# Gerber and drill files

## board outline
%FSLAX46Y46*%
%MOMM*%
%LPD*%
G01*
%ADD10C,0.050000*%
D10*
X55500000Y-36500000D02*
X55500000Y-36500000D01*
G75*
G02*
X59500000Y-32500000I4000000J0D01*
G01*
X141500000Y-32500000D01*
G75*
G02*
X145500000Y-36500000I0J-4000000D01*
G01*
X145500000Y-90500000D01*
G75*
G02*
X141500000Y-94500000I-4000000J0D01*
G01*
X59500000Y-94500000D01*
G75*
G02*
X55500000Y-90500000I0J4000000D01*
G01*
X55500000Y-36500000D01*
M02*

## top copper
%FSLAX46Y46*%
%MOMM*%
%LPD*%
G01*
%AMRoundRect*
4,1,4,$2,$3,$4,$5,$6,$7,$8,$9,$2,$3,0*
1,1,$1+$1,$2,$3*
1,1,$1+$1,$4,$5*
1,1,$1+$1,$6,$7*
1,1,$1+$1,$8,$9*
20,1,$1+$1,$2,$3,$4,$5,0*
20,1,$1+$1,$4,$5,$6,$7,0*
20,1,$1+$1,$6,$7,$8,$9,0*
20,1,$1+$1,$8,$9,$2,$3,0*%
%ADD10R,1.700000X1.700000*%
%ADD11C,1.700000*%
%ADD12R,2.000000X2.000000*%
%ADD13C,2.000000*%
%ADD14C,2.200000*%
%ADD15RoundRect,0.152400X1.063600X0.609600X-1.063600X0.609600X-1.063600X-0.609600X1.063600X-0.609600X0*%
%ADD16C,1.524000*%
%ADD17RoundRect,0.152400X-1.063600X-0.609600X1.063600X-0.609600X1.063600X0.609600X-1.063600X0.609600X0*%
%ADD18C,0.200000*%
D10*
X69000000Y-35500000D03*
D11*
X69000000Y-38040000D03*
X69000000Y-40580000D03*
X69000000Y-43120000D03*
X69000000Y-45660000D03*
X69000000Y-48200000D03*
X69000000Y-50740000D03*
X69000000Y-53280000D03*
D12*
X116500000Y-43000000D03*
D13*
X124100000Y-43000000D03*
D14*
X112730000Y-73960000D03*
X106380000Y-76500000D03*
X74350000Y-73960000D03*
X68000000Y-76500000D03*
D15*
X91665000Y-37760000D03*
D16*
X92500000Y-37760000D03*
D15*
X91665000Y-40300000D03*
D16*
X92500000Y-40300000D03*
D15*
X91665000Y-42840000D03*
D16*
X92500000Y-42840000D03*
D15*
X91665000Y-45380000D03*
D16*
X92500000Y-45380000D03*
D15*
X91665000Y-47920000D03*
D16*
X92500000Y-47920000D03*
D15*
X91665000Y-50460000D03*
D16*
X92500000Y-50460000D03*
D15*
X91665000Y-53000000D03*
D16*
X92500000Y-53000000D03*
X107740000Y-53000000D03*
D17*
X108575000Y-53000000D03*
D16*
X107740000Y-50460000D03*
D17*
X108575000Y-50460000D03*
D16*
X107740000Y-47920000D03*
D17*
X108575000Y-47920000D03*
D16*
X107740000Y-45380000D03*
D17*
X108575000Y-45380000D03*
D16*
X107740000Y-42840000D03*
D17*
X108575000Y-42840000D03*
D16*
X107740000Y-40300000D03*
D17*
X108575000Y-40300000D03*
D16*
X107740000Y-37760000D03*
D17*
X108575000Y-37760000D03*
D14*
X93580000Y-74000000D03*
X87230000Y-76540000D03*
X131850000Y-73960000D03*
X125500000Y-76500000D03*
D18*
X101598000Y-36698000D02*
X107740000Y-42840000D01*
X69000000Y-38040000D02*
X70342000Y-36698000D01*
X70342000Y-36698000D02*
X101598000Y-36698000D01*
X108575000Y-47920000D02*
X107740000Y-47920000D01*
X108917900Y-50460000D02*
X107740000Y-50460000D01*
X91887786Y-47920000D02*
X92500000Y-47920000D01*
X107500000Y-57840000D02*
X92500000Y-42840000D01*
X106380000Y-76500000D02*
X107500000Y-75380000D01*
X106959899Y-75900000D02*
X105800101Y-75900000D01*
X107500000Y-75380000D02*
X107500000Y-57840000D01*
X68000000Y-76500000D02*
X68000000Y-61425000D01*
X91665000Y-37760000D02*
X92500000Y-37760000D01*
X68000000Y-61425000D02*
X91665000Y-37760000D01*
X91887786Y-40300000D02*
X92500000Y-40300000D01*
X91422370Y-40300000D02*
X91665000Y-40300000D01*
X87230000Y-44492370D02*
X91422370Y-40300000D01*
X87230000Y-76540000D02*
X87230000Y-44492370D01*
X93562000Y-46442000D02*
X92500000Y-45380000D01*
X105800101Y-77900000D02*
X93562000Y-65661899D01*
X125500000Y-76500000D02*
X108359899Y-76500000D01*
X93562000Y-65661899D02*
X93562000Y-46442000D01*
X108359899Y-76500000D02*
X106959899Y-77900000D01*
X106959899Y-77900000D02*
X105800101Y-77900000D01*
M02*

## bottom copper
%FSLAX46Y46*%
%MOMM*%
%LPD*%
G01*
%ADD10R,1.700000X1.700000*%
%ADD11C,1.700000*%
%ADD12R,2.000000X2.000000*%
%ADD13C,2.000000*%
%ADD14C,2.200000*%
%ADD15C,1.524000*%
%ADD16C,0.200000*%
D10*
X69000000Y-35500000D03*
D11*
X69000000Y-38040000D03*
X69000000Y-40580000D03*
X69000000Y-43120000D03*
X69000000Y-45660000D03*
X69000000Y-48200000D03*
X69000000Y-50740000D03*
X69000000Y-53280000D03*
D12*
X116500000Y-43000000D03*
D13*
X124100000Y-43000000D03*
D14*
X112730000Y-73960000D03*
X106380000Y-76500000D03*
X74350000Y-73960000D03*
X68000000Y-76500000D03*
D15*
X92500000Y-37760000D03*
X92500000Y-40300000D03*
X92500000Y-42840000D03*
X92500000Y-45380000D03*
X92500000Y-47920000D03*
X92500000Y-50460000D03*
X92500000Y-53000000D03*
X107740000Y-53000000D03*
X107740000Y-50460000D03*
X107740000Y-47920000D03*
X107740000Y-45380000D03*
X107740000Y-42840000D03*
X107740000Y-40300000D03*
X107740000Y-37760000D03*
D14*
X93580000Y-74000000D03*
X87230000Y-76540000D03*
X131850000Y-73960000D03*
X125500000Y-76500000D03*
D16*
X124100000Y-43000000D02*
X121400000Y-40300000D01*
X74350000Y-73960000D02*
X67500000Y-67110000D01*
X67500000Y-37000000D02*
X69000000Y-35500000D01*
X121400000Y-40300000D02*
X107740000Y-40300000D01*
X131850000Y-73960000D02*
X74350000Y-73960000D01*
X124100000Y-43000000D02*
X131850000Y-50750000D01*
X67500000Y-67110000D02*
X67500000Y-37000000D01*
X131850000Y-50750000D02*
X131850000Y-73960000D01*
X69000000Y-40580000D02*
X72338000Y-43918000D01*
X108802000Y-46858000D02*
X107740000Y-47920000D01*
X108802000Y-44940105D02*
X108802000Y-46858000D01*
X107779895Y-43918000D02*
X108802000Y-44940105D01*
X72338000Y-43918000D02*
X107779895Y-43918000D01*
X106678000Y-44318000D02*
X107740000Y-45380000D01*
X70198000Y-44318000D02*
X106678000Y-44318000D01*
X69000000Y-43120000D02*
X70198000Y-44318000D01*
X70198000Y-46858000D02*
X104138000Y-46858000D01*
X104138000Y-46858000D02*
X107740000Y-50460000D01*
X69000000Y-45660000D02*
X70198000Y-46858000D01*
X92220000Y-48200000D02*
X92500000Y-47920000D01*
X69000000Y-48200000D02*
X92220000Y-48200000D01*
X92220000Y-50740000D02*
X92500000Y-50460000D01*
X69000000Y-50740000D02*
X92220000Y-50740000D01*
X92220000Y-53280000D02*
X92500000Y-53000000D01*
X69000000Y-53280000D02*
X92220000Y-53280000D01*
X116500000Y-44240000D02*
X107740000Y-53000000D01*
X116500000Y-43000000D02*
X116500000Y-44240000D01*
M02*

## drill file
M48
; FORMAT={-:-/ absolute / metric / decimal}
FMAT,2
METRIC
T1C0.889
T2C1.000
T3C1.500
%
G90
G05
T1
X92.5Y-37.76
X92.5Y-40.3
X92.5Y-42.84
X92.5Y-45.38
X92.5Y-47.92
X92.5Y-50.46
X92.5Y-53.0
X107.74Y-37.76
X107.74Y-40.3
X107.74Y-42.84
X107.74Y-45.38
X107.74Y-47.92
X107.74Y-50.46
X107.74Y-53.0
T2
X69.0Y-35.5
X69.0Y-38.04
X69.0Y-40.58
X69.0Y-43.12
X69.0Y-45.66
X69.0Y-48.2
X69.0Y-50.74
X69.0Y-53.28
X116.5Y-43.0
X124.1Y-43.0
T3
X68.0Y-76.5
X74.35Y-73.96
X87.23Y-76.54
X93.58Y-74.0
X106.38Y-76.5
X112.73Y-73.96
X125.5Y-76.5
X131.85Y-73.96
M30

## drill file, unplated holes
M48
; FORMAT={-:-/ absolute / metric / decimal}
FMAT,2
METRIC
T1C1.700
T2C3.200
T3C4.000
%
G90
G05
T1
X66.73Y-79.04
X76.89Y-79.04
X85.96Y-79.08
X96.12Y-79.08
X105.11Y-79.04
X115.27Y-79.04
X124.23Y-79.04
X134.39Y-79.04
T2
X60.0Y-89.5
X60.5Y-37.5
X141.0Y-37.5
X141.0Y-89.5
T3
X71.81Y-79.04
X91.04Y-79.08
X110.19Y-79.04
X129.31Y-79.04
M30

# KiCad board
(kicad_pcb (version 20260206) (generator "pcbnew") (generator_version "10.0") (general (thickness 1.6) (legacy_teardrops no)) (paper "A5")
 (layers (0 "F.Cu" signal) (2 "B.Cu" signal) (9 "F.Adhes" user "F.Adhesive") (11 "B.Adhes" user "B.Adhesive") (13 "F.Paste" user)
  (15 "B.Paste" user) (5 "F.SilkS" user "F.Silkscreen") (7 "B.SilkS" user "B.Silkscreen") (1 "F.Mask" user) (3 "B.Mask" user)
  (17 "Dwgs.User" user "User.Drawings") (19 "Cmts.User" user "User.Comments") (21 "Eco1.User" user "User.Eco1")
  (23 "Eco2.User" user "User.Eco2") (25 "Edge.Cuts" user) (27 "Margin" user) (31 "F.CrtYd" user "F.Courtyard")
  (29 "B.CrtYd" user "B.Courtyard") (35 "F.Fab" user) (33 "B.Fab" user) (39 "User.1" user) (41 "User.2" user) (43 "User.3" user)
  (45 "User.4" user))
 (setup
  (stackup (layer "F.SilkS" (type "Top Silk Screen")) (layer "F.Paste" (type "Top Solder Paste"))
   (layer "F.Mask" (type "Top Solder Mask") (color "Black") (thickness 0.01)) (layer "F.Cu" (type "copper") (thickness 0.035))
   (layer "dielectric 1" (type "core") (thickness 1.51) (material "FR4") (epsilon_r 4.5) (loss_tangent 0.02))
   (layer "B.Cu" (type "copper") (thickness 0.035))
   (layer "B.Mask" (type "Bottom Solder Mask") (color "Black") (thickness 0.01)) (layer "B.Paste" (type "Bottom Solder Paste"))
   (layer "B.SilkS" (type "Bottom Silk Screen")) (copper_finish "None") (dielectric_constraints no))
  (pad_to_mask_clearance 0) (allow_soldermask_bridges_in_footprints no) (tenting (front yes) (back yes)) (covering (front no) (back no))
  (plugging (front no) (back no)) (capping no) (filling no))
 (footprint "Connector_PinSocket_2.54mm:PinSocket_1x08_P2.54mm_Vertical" (layer "F.Cu") (at 69 35.5)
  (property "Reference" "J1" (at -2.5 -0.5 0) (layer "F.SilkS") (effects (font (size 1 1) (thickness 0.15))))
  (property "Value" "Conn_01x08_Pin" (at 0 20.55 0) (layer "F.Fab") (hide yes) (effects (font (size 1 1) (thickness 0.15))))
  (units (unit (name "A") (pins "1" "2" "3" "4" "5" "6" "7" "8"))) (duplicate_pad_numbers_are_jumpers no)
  (pad "1" thru_hole rect (at 0 0) (size 1.7 1.7) (drill 1) (layers "*.Cu" "*.Mask") (remove_unused_layers no) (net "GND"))
  (pad "2" thru_hole circle (at 0 2.54) (size 1.7 1.7) (drill 1) (layers "*.Cu" "*.Mask") (remove_unused_layers no) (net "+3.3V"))
  (pad "3" thru_hole circle (at 0 5.08) (size 1.7 1.7) (drill 1) (layers "*.Cu" "*.Mask") (remove_unused_layers no) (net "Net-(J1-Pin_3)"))
  (pad "4" thru_hole circle (at 0 7.62) (size 1.7 1.7) (drill 1) (layers "*.Cu" "*.Mask") (remove_unused_layers no) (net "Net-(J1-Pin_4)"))
  (pad "5" thru_hole circle (at 0 10.16) (size 1.7 1.7) (drill 1) (layers "*.Cu" "*.Mask") (remove_unused_layers no) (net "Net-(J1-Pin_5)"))
  (pad "6" thru_hole circle (at 0 12.7) (size 1.7 1.7) (drill 1) (layers "*.Cu" "*.Mask") (remove_unused_layers no) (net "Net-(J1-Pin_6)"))
  (pad "7" thru_hole circle (at 0 15.24) (size 1.7 1.7) (drill 1) (layers "*.Cu" "*.Mask") (remove_unused_layers no) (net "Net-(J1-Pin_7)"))
  (pad "8" thru_hole circle (at 0 17.78) (size 1.7 1.7) (drill 1) (layers "*.Cu" "*.Mask") (remove_unused_layers no) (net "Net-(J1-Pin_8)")))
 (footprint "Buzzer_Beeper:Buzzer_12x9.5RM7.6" (layer "F.Cu") (at 116.5 43)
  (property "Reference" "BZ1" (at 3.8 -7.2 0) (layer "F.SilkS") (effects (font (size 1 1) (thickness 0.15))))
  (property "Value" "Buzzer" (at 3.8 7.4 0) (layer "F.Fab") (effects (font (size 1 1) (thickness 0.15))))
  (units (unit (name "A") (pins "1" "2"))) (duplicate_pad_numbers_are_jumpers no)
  (pad "1" thru_hole rect (at 0 0) (size 2 2) (drill 1) (layers "*.Cu" "*.Mask") (remove_unused_layers no) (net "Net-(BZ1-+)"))
  (pad "2" thru_hole circle (at 7.6 0) (size 2 2) (drill 1) (layers "*.Cu" "*.Mask") (remove_unused_layers no) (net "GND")))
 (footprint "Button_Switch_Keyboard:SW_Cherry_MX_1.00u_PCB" (layer "F.Cu") (at 112.73 73.96)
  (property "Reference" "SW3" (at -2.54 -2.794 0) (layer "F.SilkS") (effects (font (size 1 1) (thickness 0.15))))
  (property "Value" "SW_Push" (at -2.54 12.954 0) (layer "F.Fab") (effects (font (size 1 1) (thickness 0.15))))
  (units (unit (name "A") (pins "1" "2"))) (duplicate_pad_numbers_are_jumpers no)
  (pad "" np_thru_hole circle (at -7.62 5.08) (size 1.7 1.7) (drill 1.7) (layers "*.Cu" "*.Mask"))
  (pad "" np_thru_hole circle (at -2.54 5.08) (size 4 4) (drill 4) (layers "*.Cu" "*.Mask"))
  (pad "" np_thru_hole circle (at 2.54 5.08) (size 1.7 1.7) (drill 1.7) (layers "*.Cu" "*.Mask"))
  (pad "1" thru_hole circle (at 0 0) (size 2.2 2.2) (drill 1.5) (layers "*.Cu" "*.Mask") (remove_unused_layers no) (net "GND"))
  (pad "2" thru_hole circle (at -6.35 2.54) (size 2.2 2.2) (drill 1.5) (layers "*.Cu" "*.Mask") (remove_unused_layers no)
   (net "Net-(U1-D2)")))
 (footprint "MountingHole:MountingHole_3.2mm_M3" (layer "F.Cu") (at 141 89.5)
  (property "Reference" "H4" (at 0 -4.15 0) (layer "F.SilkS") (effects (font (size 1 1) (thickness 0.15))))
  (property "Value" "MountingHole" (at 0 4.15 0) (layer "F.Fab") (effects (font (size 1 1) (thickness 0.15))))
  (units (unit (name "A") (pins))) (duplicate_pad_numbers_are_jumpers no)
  (pad "" np_thru_hole circle (at 0 0) (size 3.2 3.2) (drill 3.2) (layers "*.Cu" "*.Mask")))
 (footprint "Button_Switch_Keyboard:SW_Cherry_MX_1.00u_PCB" (layer "F.Cu") (at 74.35 73.96)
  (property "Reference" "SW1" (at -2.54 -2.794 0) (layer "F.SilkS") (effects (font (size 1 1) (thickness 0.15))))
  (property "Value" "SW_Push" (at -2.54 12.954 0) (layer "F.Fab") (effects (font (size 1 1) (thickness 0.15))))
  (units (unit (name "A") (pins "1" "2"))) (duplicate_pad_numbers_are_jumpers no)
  (pad "" np_thru_hole circle (at -7.62 5.08) (size 1.7 1.7) (drill 1.7) (layers "*.Cu" "*.Mask"))
  (pad "" np_thru_hole circle (at -2.54 5.08) (size 4 4) (drill 4) (layers "*.Cu" "*.Mask"))
  (pad "" np_thru_hole circle (at 2.54 5.08) (size 1.7 1.7) (drill 1.7) (layers "*.Cu" "*.Mask"))
  (pad "1" thru_hole circle (at 0 0) (size 2.2 2.2) (drill 1.5) (layers "*.Cu" "*.Mask") (remove_unused_layers no) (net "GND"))
  (pad "2" thru_hole circle (at -6.35 2.54) (size 2.2 2.2) (drill 1.5) (layers "*.Cu" "*.Mask") (remove_unused_layers no)
   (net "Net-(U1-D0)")))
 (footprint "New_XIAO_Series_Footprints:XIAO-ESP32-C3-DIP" (layer "F.Cu") (at 100.12 45.38 90)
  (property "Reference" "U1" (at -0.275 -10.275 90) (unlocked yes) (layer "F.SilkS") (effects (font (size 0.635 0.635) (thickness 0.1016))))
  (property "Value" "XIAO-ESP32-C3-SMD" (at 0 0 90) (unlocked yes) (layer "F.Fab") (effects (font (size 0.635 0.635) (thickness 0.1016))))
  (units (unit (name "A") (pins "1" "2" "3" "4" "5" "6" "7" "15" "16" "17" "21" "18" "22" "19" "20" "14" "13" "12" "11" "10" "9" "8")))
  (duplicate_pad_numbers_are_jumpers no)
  (pad "1" smd roundrect (at 7.62 -8.455 180) (size 2.432 1.524) (layers "F.Cu" "F.Mask") (roundrect_rratio 0.1) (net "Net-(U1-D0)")
   (thermal_bridge_angle 45))
  (pad "1" thru_hole circle (at 7.62 -7.62 180) (size 1.524 1.524) (drill 0.889) (layers "*.Cu" "*.Mask") (remove_unused_layers no)
   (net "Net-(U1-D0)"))
  (pad "2" smd roundrect (at 5.08 -8.455 180) (size 2.432 1.524) (layers "F.Cu" "F.Mask") (roundrect_rratio 0.1) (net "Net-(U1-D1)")
   (thermal_bridge_angle 45))
  (pad "2" thru_hole circle (at 5.08 -7.62 180) (size 1.524 1.524) (drill 0.889) (layers "*.Cu" "*.Mask") (remove_unused_layers no)
   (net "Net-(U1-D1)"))
  (pad "3" smd roundrect (at 2.54 -8.455 180) (size 2.432 1.524) (layers "F.Cu" "F.Mask") (roundrect_rratio 0.1) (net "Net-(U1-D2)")
   (thermal_bridge_angle 45))
  (pad "3" thru_hole circle (at 2.54 -7.62 180) (size 1.524 1.524) (drill 0.889) (layers "*.Cu" "*.Mask") (remove_unused_layers no)
   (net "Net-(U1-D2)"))
  (pad "4" smd roundrect (at 0 -8.455 180) (size 2.432 1.524) (layers "F.Cu" "F.Mask") (roundrect_rratio 0.1) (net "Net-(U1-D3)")
   (thermal_bridge_angle 45))
  (pad "4" thru_hole circle (at 0 -7.62 180) (size 1.524 1.524) (drill 0.889) (layers "*.Cu" "*.Mask") (remove_unused_layers no)
   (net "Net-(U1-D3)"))
  (pad "5" smd roundrect (at -2.54 -8.455 180) (size 2.432 1.524) (layers "F.Cu" "F.Mask") (roundrect_rratio 0.1) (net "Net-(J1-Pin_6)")
   (thermal_bridge_angle 45))
  (pad "5" thru_hole circle (at -2.54 -7.62 180) (size 1.524 1.524) (drill 0.889) (layers "*.Cu" "*.Mask") (remove_unused_layers no)
   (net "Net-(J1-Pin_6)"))
  (pad "6" smd roundrect (at -5.08 -8.455 180) (size 2.432 1.524) (layers "F.Cu" "F.Mask") (roundrect_rratio 0.1) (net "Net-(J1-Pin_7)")
   (thermal_bridge_angle 45))
  (pad "6" thru_hole circle (at -5.08 -7.62 180) (size 1.524 1.524) (drill 0.889) (layers "*.Cu" "*.Mask") (remove_unused_layers no)
   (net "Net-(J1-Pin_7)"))
  (pad "7" smd roundrect (at -7.62 -8.455 180) (size 2.432 1.524) (layers "F.Cu" "F.Mask") (roundrect_rratio 0.1) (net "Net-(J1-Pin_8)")
   (thermal_bridge_angle 45))
  (pad "7" thru_hole circle (at -7.62 -7.62 180) (size 1.524 1.524) (drill 0.889) (layers "*.Cu" "*.Mask") (remove_unused_layers no)
   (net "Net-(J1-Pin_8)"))
  (pad "8" thru_hole circle (at -7.62 7.62) (size 1.524 1.524) (drill 0.889) (layers "*.Cu" "*.Mask") (remove_unused_layers no)
   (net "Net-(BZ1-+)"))
  (pad "8" smd roundrect (at -7.62 8.455) (size 2.432 1.524) (layers "F.Cu" "F.Mask") (roundrect_rratio 0.1) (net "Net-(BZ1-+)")
   (thermal_bridge_angle 45))
  (pad "9" thru_hole circle (at -5.08 7.62) (size 1.524 1.524) (drill 0.889) (layers "*.Cu" "*.Mask") (remove_unused_layers no)
   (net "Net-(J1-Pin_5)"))
  (pad "9" smd roundrect (at -5.08 8.455) (size 2.432 1.524) (layers "F.Cu" "F.Mask") (roundrect_rratio 0.1) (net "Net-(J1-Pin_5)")
   (thermal_bridge_angle 45))
  (pad "10" thru_hole circle (at -2.54 7.62) (size 1.524 1.524) (drill 0.889) (layers "*.Cu" "*.Mask") (remove_unused_layers no)
   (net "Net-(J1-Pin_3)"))
  (pad "10" smd roundrect (at -2.54 8.455) (size 2.432 1.524) (layers "F.Cu" "F.Mask") (roundrect_rratio 0.1) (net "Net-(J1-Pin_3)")
   (thermal_bridge_angle 45))
  (pad "11" thru_hole circle (at 0 7.62) (size 1.524 1.524) (drill 0.889) (layers "*.Cu" "*.Mask") (remove_unused_layers no)
   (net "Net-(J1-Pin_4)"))
  (pad "11" smd roundrect (at 0 8.455) (size 2.432 1.524) (layers "F.Cu" "F.Mask") (roundrect_rratio 0.1) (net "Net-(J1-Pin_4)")
   (thermal_bridge_angle 45))
  (pad "12" thru_hole circle (at 2.54 7.62) (size 1.524 1.524) (drill 0.889) (layers "*.Cu" "*.Mask") (remove_unused_layers no)
   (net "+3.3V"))
  (pad "12" smd roundrect (at 2.54 8.455) (size 2.432 1.524) (layers "F.Cu" "F.Mask") (roundrect_rratio 0.1) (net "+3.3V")
   (thermal_bridge_angle 45))
  (pad "13" thru_hole circle (at 5.08 7.62) (size 1.524 1.524) (drill 0.889) (layers "*.Cu" "*.Mask") (remove_unused_layers no) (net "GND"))
  (pad "13" smd roundrect (at 5.08 8.455) (size 2.432 1.524) (layers "F.Cu" "F.Mask") (roundrect_rratio 0.1) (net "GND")
   (thermal_bridge_angle 45))
  (pad "14" thru_hole circle (at 7.62 7.62) (size 1.524 1.524) (drill 0.889) (layers "*.Cu" "*.Mask") (remove_unused_layers no)
   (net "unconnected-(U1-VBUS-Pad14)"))
  (pad "14" smd roundrect (at 7.62 8.455) (size 2.432 1.524) (layers "F.Cu" "F.Mask") (roundrect_rratio 0.1)
   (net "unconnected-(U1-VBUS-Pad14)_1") (thermal_bridge_angle 45)))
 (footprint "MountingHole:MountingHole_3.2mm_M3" (layer "F.Cu") (at 141 37.5)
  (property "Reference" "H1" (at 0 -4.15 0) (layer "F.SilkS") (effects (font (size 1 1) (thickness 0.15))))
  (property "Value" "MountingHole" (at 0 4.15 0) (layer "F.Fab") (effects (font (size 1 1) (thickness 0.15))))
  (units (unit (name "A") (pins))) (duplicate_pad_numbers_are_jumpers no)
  (pad "" np_thru_hole circle (at 0 0) (size 3.2 3.2) (drill 3.2) (layers "*.Cu" "*.Mask")))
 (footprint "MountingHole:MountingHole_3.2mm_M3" (layer "F.Cu") (at 60.5 37.5)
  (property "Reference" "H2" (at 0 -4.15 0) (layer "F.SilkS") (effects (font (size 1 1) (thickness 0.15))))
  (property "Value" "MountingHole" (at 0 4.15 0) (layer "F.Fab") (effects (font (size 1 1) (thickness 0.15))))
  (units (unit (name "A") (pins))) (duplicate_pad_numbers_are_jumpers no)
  (pad "" np_thru_hole circle (at 0 0) (size 3.2 3.2) (drill 3.2) (layers "*.Cu" "*.Mask")))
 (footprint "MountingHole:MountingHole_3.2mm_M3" (layer "F.Cu") (at 60 89.5)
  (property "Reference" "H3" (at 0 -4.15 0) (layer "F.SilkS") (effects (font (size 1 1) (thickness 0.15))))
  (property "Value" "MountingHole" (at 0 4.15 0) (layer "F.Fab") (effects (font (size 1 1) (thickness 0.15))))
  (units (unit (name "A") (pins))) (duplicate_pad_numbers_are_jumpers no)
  (pad "" np_thru_hole circle (at 0 0) (size 3.2 3.2) (drill 3.2) (layers "*.Cu" "*.Mask")))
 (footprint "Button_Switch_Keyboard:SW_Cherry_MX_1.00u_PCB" (layer "F.Cu") (at 93.58 74)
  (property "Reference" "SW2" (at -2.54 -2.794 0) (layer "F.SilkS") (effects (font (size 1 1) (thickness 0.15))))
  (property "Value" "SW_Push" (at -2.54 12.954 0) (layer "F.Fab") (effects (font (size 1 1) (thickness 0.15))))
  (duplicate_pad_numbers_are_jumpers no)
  (pad "" np_thru_hole circle (at -7.62 5.08) (size 1.7 1.7) (drill 1.7) (layers "*.Cu" "*.Mask"))
  (pad "" np_thru_hole circle (at -2.54 5.08) (size 4 4) (drill 4) (layers "*.Cu" "*.Mask"))
  (pad "" np_thru_hole circle (at 2.54 5.08) (size 1.7 1.7) (drill 1.7) (layers "*.Cu" "*.Mask"))
  (pad "1" thru_hole circle (at 0 0) (size 2.2 2.2) (drill 1.5) (layers "*.Cu" "*.Mask") (remove_unused_layers no) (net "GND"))
  (pad "2" thru_hole circle (at -6.35 2.54) (size 2.2 2.2) (drill 1.5) (layers "*.Cu" "*.Mask") (remove_unused_layers no)
   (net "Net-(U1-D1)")))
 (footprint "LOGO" (layer "F.Cu") (at 134.5 58.5)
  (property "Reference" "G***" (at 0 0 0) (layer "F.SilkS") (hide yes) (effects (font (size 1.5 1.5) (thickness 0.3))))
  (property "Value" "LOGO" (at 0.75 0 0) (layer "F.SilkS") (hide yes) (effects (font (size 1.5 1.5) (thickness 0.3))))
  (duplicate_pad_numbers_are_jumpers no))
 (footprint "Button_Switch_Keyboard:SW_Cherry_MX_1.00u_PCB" (layer "F.Cu") (at 131.85 73.96)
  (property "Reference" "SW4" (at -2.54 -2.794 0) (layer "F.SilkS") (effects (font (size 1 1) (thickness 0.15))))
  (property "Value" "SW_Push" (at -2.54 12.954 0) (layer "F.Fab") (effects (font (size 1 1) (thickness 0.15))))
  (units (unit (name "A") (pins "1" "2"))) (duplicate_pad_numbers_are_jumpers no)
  (pad "" np_thru_hole circle (at -7.62 5.08) (size 1.7 1.7) (drill 1.7) (layers "*.Cu" "*.Mask"))
  (pad "" np_thru_hole circle (at -2.54 5.08) (size 4 4) (drill 4) (layers "*.Cu" "*.Mask"))
  (pad "" np_thru_hole circle (at 2.54 5.08) (size 1.7 1.7) (drill 1.7) (layers "*.Cu" "*.Mask"))
  (pad "1" thru_hole circle (at 0 0) (size 2.2 2.2) (drill 1.5) (layers "*.Cu" "*.Mask") (remove_unused_layers no) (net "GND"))
  (pad "2" thru_hole circle (at -6.35 2.54) (size 2.2 2.2) (drill 1.5) (layers "*.Cu" "*.Mask") (remove_unused_layers no)
   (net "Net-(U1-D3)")))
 (gr_rect (start 55.5 32.5) (end 145.5 94.5) (radius 4) (stroke (width 0.05) (type solid)) (fill no) (layer "Edge.Cuts"))
 (segment (start 124.1 43) (end 121.4 40.3) (width 0.2) (layer "B.Cu") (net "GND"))
 (segment (start 74.35 73.96) (end 67.5 67.11) (width 0.2) (layer "B.Cu") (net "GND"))
 (segment (start 67.5 37) (end 69 35.5) (width 0.2) (layer "B.Cu") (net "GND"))
 (segment (start 121.4 40.3) (end 107.74 40.3) (width 0.2) (layer "B.Cu") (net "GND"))
 (segment (start 131.85 73.96) (end 74.35 73.96) (width 0.2) (layer "B.Cu") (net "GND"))
 (segment (start 124.1 43) (end 131.85 50.75) (width 0.2) (layer "B.Cu") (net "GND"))
 (segment (start 67.5 67.11) (end 67.5 37) (width 0.2) (layer "B.Cu") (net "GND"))
 (segment (start 131.85 50.75) (end 131.85 73.96) (width 0.2) (layer "B.Cu") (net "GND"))
 (segment (start 101.598 36.698) (end 107.74 42.84) (width 0.2) (layer "F.Cu") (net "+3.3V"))
 (segment (start 69 38.04) (end 70.342 36.698) (width 0.2) (layer "F.Cu") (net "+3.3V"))
 (segment (start 70.342 36.698) (end 101.598 36.698) (width 0.2) (layer "F.Cu") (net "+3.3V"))
 (segment (start 108.575 47.92) (end 107.74 47.92) (width 0.2) (layer "F.Cu") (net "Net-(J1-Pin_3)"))
 (segment (start 69 40.58) (end 72.338 43.918) (width 0.2) (layer "B.Cu") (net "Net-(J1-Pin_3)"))
 (segment (start 108.802 46.858) (end 107.74 47.92) (width 0.2) (layer "B.Cu") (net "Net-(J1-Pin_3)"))
 (segment (start 108.802 44.940105) (end 108.802 46.858) (width 0.2) (layer "B.Cu") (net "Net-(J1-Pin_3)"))
 (segment (start 107.779895 43.918) (end 108.802 44.940105) (width 0.2) (layer "B.Cu") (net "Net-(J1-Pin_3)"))
 (segment (start 72.338 43.918) (end 107.779895 43.918) (width 0.2) (layer "B.Cu") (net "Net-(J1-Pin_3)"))
 (segment (start 106.678 44.318) (end 107.74 45.38) (width 0.2) (layer "B.Cu") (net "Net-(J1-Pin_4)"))
 (segment (start 70.198 44.318) (end 106.678 44.318) (width 0.2) (layer "B.Cu") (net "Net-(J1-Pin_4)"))
 (segment (start 69 43.12) (end 70.198 44.318) (width 0.2) (layer "B.Cu") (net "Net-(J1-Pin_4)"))
 (segment (start 108.9179 50.46) (end 107.74 50.46) (width 0.2) (layer "F.Cu") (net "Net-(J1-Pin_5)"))
 (segment (start 70.198 46.858) (end 104.138 46.858) (width 0.2) (layer "B.Cu") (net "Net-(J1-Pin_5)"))
 (segment (start 104.138 46.858) (end 107.74 50.46) (width 0.2) (layer "B.Cu") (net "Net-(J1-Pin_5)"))
 (segment (start 69 45.66) (end 70.198 46.858) (width 0.2) (layer "B.Cu") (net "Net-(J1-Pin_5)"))
 (segment (start 91.887786 47.92) (end 92.5 47.92) (width 0.2) (layer "F.Cu") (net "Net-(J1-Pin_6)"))
 (segment (start 92.22 48.2) (end 92.5 47.92) (width 0.2) (layer "B.Cu") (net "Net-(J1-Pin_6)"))
 (segment (start 69 48.2) (end 92.22 48.2) (width 0.2) (layer "B.Cu") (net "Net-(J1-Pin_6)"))
 (segment (start 92.22 50.74) (end 92.5 50.46) (width 0.2) (layer "B.Cu") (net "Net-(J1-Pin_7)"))
 (segment (start 69 50.74) (end 92.22 50.74) (width 0.2) (layer "B.Cu") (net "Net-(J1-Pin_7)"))
 (segment (start 92.22 53.28) (end 92.5 53) (width 0.2) (layer "B.Cu") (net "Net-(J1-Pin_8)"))
 (segment (start 69 53.28) (end 92.22 53.28) (width 0.2) (layer "B.Cu") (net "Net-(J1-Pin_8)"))
 (segment (start 116.5 44.24) (end 107.74 53) (width 0.2) (layer "B.Cu") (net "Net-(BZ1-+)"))
 (segment (start 116.5 43) (end 116.5 44.24) (width 0.2) (layer "B.Cu") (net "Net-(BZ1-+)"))
 (segment (start 107.5 57.84) (end 92.5 42.84) (width 0.2) (layer "F.Cu") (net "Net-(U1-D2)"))
 (segment (start 106.38 76.5) (end 107.5 75.38) (width 0.2) (layer "F.Cu") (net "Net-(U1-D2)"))
 (segment (start 106.959899 75.9) (end 105.800101 75.9) (width 0.2) (layer "F.Cu") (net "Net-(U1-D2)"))
 (segment (start 107.5 75.38) (end 107.5 57.84) (width 0.2) (layer "F.Cu") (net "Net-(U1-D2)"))
 (segment (start 68 76.5) (end 68 61.425) (width 0.2) (layer "F.Cu") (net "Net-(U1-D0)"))
 (segment (start 91.665 37.76) (end 92.5 37.76) (width 0.2) (layer "F.Cu") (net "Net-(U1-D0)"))
 (segment (start 68 61.425) (end 91.665 37.76) (width 0.2) (layer "F.Cu") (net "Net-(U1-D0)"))
 (segment (start 91.887786 40.3) (end 92.5 40.3) (width 0.2) (layer "F.Cu") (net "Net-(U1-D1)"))
 (segment (start 91.42237 40.3) (end 91.665 40.3) (width 0.2) (layer "F.Cu") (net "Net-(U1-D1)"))
 (segment (start 87.23 44.49237) (end 91.42237 40.3) (width 0.2) (layer "F.Cu") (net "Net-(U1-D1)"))
 (segment (start 87.23 76.54) (end 87.23 44.49237) (width 0.2) (layer "F.Cu") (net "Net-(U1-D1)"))
 (segment (start 93.562 46.442) (end 92.5 45.38) (width 0.2) (layer "F.Cu") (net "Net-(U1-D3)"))
 (segment (start 105.800101 77.9) (end 93.562 65.661899) (width 0.2) (layer "F.Cu") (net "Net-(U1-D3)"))
 (segment (start 125.5 76.5) (end 108.359899 76.5) (width 0.2) (layer "F.Cu") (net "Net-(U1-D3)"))
 (segment (start 93.562 65.661899) (end 93.562 46.442) (width 0.2) (layer "F.Cu") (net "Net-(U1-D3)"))
 (segment (start 108.359899 76.5) (end 106.959899 77.9) (width 0.2) (layer "F.Cu") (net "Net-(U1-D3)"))
 (segment (start 106.959899 77.9) (end 105.800101 77.9) (width 0.2) (layer "F.Cu") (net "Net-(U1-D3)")))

